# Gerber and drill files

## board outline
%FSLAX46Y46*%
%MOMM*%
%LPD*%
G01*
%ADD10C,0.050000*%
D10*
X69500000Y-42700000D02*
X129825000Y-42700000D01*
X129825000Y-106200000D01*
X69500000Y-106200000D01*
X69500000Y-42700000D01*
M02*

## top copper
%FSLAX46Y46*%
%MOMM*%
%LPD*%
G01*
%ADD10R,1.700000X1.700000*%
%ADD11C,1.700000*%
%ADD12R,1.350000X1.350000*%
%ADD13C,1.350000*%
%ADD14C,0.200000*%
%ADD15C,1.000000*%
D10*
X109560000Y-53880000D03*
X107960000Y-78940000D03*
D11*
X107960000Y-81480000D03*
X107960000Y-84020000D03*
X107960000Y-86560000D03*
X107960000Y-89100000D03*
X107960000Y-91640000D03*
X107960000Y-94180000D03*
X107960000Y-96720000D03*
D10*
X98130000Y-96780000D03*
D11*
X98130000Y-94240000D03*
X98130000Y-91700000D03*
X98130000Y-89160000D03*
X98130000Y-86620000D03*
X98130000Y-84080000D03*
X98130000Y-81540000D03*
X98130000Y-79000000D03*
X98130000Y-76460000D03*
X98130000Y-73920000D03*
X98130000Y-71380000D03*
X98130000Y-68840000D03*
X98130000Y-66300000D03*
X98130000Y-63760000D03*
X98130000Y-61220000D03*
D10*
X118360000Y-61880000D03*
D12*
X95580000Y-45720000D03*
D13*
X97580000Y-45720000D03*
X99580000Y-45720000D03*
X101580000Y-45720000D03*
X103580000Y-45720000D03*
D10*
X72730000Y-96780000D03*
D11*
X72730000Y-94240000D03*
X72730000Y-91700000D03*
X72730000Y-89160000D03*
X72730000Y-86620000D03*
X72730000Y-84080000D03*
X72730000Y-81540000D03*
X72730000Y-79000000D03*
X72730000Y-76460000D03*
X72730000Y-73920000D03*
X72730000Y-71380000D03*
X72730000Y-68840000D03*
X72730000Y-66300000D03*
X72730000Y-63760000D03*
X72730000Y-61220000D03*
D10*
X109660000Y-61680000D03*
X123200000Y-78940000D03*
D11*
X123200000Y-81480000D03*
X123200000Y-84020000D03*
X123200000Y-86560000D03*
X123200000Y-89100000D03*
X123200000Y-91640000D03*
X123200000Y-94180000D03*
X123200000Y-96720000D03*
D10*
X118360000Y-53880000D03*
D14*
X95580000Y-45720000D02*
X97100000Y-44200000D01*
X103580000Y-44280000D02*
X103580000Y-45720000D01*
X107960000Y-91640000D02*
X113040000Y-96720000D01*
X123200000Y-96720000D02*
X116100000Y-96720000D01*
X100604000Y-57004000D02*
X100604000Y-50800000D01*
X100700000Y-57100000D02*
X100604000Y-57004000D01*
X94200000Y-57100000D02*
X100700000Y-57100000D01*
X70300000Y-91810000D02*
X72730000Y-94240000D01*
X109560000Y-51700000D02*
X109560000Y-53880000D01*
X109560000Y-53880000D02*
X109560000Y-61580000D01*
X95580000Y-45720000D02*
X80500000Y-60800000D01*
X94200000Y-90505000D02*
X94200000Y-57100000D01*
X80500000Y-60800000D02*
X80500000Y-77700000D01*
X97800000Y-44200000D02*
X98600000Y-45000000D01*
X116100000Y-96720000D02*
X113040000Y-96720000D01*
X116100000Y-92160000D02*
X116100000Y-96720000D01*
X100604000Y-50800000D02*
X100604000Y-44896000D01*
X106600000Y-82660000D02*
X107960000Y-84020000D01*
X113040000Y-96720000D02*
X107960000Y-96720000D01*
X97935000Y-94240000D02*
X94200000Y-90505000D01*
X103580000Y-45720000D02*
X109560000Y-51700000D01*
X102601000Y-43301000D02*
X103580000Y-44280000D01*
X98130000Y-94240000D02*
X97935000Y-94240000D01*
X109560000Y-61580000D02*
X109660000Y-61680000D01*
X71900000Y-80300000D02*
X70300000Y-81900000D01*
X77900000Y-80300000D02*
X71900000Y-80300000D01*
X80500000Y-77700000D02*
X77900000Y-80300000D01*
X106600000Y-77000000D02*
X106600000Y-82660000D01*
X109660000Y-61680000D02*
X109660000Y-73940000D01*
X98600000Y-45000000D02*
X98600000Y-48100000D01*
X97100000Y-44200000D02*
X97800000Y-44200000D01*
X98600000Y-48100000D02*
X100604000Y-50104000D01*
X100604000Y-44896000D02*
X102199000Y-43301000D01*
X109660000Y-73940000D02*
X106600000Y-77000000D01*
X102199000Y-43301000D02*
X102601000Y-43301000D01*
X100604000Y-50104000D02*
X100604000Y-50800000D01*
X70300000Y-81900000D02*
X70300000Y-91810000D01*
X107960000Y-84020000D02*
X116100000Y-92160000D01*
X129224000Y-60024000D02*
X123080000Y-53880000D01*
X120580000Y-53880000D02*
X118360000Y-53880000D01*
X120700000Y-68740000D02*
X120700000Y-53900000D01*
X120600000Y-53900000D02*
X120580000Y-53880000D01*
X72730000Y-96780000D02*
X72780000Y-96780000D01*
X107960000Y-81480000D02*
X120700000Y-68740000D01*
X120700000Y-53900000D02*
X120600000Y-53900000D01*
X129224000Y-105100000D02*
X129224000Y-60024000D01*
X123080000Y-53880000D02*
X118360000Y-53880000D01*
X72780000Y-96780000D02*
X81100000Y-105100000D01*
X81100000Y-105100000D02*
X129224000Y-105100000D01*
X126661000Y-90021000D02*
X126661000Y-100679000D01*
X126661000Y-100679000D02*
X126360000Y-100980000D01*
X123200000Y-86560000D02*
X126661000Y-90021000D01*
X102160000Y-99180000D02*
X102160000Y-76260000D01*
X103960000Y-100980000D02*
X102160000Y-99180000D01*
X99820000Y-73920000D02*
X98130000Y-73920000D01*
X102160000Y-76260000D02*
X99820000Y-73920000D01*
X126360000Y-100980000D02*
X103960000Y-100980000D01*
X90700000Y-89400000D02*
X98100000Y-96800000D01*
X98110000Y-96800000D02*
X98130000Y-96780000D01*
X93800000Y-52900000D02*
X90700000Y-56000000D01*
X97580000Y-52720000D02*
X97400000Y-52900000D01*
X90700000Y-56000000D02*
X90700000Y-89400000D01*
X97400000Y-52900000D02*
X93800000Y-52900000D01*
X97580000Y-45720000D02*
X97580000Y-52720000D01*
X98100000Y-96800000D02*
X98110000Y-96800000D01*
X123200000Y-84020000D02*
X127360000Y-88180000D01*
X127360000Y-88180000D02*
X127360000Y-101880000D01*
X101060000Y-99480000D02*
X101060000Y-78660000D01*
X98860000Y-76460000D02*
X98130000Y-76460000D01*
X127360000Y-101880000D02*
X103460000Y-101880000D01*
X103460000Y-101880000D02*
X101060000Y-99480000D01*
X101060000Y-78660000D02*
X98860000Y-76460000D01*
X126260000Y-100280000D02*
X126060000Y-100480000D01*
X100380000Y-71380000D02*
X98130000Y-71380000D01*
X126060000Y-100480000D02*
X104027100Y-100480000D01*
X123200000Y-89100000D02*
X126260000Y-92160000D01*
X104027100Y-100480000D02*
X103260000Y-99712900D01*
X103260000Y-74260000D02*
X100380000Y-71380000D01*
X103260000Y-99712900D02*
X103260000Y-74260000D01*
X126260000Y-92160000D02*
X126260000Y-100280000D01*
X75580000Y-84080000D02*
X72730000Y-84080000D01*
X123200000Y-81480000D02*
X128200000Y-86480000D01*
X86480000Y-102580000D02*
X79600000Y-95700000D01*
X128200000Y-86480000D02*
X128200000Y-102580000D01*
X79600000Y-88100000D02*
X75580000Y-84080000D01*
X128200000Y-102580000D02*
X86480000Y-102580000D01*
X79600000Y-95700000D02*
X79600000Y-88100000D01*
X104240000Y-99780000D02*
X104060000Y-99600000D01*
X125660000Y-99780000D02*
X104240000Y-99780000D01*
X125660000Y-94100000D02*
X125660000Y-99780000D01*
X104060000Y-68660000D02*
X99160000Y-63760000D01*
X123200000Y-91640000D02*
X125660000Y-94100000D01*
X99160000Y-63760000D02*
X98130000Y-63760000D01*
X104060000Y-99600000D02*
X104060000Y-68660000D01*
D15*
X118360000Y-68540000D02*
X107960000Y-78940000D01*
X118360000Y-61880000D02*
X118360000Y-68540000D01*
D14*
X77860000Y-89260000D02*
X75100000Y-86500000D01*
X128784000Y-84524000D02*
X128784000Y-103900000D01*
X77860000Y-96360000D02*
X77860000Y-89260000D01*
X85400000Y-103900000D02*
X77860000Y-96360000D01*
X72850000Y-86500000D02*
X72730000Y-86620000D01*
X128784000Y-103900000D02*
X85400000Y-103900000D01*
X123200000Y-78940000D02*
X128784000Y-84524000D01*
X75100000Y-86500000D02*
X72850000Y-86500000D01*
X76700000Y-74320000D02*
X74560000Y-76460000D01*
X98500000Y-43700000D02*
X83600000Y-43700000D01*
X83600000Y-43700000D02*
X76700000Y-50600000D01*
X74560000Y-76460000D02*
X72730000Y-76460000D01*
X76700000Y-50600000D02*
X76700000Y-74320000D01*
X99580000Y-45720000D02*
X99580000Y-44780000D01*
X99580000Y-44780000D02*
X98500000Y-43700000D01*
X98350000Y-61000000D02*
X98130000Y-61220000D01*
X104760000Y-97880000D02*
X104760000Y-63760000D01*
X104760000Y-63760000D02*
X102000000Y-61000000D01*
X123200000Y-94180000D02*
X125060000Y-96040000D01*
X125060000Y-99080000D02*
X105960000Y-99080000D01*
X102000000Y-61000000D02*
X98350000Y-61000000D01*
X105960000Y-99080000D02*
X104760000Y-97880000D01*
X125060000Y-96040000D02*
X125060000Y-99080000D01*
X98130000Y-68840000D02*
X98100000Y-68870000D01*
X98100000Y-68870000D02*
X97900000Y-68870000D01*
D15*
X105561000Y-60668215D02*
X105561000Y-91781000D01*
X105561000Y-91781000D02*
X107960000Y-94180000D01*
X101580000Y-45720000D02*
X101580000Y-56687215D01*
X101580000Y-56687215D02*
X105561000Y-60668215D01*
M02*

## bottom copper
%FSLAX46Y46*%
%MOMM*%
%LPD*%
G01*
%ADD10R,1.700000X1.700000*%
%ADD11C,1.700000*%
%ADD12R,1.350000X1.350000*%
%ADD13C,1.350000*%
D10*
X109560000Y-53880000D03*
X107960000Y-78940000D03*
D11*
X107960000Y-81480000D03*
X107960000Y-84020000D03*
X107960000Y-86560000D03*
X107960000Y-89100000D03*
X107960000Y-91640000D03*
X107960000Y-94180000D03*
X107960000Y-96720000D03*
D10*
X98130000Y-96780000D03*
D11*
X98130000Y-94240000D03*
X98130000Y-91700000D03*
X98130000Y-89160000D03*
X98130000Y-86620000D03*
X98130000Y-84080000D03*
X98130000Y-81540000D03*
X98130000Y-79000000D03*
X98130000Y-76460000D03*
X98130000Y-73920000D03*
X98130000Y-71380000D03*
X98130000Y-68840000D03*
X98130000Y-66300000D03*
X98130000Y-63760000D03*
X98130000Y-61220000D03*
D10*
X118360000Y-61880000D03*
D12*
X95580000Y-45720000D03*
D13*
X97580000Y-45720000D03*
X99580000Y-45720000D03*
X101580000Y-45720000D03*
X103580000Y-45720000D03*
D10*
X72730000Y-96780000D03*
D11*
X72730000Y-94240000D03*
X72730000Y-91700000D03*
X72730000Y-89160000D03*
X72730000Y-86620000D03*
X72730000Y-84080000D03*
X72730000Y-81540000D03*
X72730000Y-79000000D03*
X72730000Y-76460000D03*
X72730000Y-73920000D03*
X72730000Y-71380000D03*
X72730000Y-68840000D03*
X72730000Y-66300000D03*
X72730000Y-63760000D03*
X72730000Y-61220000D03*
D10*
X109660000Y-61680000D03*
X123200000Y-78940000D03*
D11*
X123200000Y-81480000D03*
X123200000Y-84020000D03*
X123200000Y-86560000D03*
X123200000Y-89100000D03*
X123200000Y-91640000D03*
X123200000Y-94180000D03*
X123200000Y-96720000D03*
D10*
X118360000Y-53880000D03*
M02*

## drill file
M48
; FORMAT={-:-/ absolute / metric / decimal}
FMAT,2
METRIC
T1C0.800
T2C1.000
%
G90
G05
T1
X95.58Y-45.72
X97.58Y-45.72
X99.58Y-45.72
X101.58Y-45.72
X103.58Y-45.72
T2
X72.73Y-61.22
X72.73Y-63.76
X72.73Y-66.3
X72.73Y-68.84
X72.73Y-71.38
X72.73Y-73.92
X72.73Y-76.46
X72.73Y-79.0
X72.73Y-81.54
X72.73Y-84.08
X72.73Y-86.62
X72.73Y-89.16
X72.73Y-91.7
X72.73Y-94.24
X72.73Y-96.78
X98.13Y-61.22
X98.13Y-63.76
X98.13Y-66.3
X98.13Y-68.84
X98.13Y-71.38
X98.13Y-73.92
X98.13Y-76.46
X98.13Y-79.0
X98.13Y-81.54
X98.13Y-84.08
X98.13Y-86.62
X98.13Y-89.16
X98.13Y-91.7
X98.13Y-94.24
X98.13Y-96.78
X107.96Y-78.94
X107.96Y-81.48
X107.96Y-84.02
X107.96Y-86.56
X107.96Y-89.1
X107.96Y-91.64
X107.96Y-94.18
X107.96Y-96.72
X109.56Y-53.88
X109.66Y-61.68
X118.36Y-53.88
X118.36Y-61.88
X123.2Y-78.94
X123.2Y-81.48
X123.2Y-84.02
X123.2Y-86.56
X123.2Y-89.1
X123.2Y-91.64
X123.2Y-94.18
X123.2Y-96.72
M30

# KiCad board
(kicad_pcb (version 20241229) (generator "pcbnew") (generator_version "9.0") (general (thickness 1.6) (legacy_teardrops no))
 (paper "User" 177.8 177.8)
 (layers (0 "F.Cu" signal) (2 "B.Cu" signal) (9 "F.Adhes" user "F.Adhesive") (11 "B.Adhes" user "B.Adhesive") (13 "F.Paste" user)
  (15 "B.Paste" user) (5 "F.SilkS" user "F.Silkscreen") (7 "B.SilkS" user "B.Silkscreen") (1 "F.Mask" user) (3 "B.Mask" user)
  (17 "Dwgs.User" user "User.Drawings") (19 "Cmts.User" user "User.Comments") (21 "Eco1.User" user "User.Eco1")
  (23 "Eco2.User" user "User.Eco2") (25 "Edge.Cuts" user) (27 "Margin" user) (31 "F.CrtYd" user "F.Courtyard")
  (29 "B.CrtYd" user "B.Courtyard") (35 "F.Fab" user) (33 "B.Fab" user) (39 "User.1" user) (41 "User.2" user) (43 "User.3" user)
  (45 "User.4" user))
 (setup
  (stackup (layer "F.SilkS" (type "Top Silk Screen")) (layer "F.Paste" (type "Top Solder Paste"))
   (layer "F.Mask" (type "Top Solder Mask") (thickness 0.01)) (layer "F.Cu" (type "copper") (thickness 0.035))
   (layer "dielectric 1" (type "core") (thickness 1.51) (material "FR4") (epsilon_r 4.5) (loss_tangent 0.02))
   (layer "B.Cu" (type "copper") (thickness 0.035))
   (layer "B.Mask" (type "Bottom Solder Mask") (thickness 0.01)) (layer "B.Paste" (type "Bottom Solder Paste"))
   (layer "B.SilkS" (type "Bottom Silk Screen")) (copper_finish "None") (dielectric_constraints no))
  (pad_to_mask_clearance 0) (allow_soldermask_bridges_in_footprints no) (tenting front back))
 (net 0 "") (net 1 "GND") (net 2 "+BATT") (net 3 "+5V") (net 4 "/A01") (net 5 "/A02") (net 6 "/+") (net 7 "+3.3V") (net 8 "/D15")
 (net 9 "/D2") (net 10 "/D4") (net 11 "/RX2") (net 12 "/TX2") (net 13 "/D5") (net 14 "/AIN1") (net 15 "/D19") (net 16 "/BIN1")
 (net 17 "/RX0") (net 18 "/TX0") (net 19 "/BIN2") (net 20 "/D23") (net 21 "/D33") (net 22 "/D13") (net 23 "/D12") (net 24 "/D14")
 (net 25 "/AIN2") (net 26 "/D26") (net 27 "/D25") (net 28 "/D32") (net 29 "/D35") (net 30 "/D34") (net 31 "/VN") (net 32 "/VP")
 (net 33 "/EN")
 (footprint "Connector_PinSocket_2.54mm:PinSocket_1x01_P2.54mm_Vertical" (layer "F.Cu") (at 109.56 53.88)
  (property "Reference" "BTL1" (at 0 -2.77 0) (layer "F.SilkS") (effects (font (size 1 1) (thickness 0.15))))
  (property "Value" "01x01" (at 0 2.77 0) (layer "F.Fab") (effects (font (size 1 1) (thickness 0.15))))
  (pad "1" thru_hole rect (at 0 0) (size 1.7 1.7) (drill 1) (layers "*.Cu" "*.Mask") (remove_unused_layers no) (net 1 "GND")))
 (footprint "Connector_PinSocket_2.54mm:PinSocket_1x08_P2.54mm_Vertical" (layer "F.Cu") (at 107.96 78.94)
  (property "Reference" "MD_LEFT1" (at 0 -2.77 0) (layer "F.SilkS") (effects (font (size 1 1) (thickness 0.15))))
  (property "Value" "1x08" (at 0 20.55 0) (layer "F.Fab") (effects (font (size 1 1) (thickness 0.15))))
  (pad "1" thru_hole rect (at 0 0) (size 1.7 1.7) (drill 1) (layers "*.Cu" "*.Mask") (remove_unused_layers no) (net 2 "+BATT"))
  (pad "2" thru_hole circle (at 0 2.54) (size 1.7 1.7) (drill 1) (layers "*.Cu" "*.Mask") (remove_unused_layers no) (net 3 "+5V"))
  (pad "3" thru_hole circle (at 0 5.08) (size 1.7 1.7) (drill 1) (layers "*.Cu" "*.Mask") (remove_unused_layers no) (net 1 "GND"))
  (pad "4" thru_hole circle (at 0 7.62) (size 1.7 1.7) (drill 1) (layers "*.Cu" "*.Mask") (remove_unused_layers no) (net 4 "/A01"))
  (pad "5" thru_hole circle (at 0 10.16) (size 1.7 1.7) (drill 1) (layers "*.Cu" "*.Mask") (remove_unused_layers no) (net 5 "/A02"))
  (pad "6" thru_hole circle (at 0 12.7) (size 1.7 1.7) (drill 1) (layers "*.Cu" "*.Mask") (remove_unused_layers no) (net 1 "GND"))
  (pad "7" thru_hole circle (at 0 15.24) (size 1.7 1.7) (drill 1) (layers "*.Cu" "*.Mask") (remove_unused_layers no) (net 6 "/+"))
  (pad "8" thru_hole circle (at 0 17.78) (size 1.7 1.7) (drill 1) (layers "*.Cu" "*.Mask") (remove_unused_layers no) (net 1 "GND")))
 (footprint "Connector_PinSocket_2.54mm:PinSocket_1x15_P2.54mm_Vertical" (layer "F.Cu") (at 98.13 96.78 180)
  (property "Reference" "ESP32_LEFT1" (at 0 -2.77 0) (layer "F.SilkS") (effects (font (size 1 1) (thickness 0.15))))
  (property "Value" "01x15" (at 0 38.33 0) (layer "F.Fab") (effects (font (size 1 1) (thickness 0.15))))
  (pad "1" thru_hole rect (at 0 0 180) (size 1.7 1.7) (drill 1) (layers "*.Cu" "*.Mask") (remove_unused_layers no) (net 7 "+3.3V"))
  (pad "2" thru_hole circle (at 0 2.54 180) (size 1.7 1.7) (drill 1) (layers "*.Cu" "*.Mask") (remove_unused_layers no) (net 1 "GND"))
  (pad "3" thru_hole circle (at 0 5.08 180) (size 1.7 1.7) (drill 1) (layers "*.Cu" "*.Mask") (remove_unused_layers no) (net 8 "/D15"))
  (pad "4" thru_hole circle (at 0 7.62 180) (size 1.7 1.7) (drill 1) (layers "*.Cu" "*.Mask") (remove_unused_layers no) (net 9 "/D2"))
  (pad "5" thru_hole circle (at 0 10.16 180) (size 1.7 1.7) (drill 1) (layers "*.Cu" "*.Mask") (remove_unused_layers no) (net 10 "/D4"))
  (pad "6" thru_hole circle (at 0 12.7 180) (size 1.7 1.7) (drill 1) (layers "*.Cu" "*.Mask") (remove_unused_layers no) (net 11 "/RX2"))
  (pad "7" thru_hole circle (at 0 15.24 180) (size 1.7 1.7) (drill 1) (layers "*.Cu" "*.Mask") (remove_unused_layers no) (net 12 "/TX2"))
  (pad "8" thru_hole circle (at 0 17.78 180) (size 1.7 1.7) (drill 1) (layers "*.Cu" "*.Mask") (remove_unused_layers no) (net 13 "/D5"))
  (pad "9" thru_hole circle (at 0 20.32 180) (size 1.7 1.7) (drill 1) (layers "*.Cu" "*.Mask") (remove_unused_layers no) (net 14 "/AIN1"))
  (pad "10" thru_hole circle (at 0 22.86 180) (size 1.7 1.7) (drill 1) (layers "*.Cu" "*.Mask") (remove_unused_layers no) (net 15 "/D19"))
  (pad "11" thru_hole circle (at 0 25.4 180) (size 1.7 1.7) (drill 1) (layers "*.Cu" "*.Mask") (remove_unused_layers no) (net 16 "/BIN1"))
  (pad "12" thru_hole circle (at 0 27.94 180) (size 1.7 1.7) (drill 1) (layers "*.Cu" "*.Mask") (remove_unused_layers no) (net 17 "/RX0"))
  (pad "13" thru_hole circle (at 0 30.48 180) (size 1.7 1.7) (drill 1) (layers "*.Cu" "*.Mask") (remove_unused_layers no) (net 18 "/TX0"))
  (pad "14" thru_hole circle (at 0 33.02 180) (size 1.7 1.7) (drill 1) (layers "*.Cu" "*.Mask") (remove_unused_layers no) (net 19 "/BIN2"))
  (pad "15" thru_hole circle (at 0 35.56 180) (size 1.7 1.7) (drill 1) (layers "*.Cu" "*.Mask") (remove_unused_layers no) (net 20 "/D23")))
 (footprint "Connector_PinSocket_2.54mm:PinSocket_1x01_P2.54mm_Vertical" (layer "F.Cu") (at 118.36 61.88)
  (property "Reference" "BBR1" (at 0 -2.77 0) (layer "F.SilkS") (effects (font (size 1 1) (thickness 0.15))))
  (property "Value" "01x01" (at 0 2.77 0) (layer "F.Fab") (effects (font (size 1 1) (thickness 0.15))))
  (pad "1" thru_hole rect (at 0 0) (size 1.7 1.7) (drill 1) (layers "*.Cu" "*.Mask") (remove_unused_layers no) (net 2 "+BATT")))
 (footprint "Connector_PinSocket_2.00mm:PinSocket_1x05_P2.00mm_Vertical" (layer "F.Cu") (at 95.58 45.72 90)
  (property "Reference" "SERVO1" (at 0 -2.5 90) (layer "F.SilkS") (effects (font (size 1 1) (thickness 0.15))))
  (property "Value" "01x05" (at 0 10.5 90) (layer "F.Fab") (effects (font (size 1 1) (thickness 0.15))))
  (pad "1" thru_hole rect (at 0 0 90) (size 1.35 1.35) (drill 0.8) (layers "*.Cu" "*.Mask") (remove_unused_layers no) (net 1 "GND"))
  (pad "2" thru_hole circle (at 0 2 90) (size 1.35 1.35) (drill 0.8) (layers "*.Cu" "*.Mask") (remove_unused_layers no) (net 7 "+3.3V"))
  (pad "3" thru_hole circle (at 0 4 90) (size 1.35 1.35) (drill 0.8) (layers "*.Cu" "*.Mask") (remove_unused_layers no) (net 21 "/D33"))
  (pad "4" thru_hole circle (at 0 6 90) (size 1.35 1.35) (drill 0.8) (layers "*.Cu" "*.Mask") (remove_unused_layers no) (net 6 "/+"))
  (pad "5" thru_hole circle (at 0 8 90) (size 1.35 1.35) (drill 0.8) (layers "*.Cu" "*.Mask") (remove_unused_layers no) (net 1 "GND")))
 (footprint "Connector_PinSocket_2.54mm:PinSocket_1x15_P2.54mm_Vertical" (layer "F.Cu") (at 72.73 96.78 180)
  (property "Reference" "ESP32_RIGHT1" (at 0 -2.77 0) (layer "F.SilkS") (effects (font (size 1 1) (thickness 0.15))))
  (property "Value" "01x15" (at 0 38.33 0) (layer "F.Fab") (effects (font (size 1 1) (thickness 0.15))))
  (pad "1" thru_hole rect (at 0 0 180) (size 1.7 1.7) (drill 1) (layers "*.Cu" "*.Mask") (remove_unused_layers no) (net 3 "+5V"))
  (pad "2" thru_hole circle (at 0 2.54 180) (size 1.7 1.7) (drill 1) (layers "*.Cu" "*.Mask") (remove_unused_layers no) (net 1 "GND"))
  (pad "3" thru_hole circle (at 0 5.08 180) (size 1.7 1.7) (drill 1) (layers "*.Cu" "*.Mask") (remove_unused_layers no) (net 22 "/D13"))
  (pad "4" thru_hole circle (at 0 7.62 180) (size 1.7 1.7) (drill 1) (layers "*.Cu" "*.Mask") (remove_unused_layers no) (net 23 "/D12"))
  (pad "5" thru_hole circle (at 0 10.16 180) (size 1.7 1.7) (drill 1) (layers "*.Cu" "*.Mask") (remove_unused_layers no) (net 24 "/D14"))
  (pad "6" thru_hole circle (at 0 12.7 180) (size 1.7 1.7) (drill 1) (layers "*.Cu" "*.Mask") (remove_unused_layers no) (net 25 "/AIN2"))
  (pad "7" thru_hole circle (at 0 15.24 180) (size 1.7 1.7) (drill 1) (layers "*.Cu" "*.Mask") (remove_unused_layers no) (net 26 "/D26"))
  (pad "8" thru_hole circle (at 0 17.78 180) (size 1.7 1.7) (drill 1) (layers "*.Cu" "*.Mask") (remove_unused_layers no) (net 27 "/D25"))
  (pad "9" thru_hole circle (at 0 20.32 180) (size 1.7 1.7) (drill 1) (layers "*.Cu" "*.Mask") (remove_unused_layers no) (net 21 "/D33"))
  (pad "10" thru_hole circle (at 0 22.86 180) (size 1.7 1.7) (drill 1) (layers "*.Cu" "*.Mask") (remove_unused_layers no) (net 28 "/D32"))
  (pad "11" thru_hole circle (at 0 25.4 180) (size 1.7 1.7) (drill 1) (layers "*.Cu" "*.Mask") (remove_unused_layers no) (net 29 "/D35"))
  (pad "12" thru_hole circle (at 0 27.94 180) (size 1.7 1.7) (drill 1) (layers "*.Cu" "*.Mask") (remove_unused_layers no) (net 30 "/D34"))
  (pad "13" thru_hole circle (at 0 30.48 180) (size 1.7 1.7) (drill 1) (layers "*.Cu" "*.Mask") (remove_unused_layers no) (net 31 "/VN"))
  (pad "14" thru_hole circle (at 0 33.02 180) (size 1.7 1.7) (drill 1) (layers "*.Cu" "*.Mask") (remove_unused_layers no) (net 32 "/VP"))
  (pad "15" thru_hole circle (at 0 35.56 180) (size 1.7 1.7) (drill 1) (layers "*.Cu" "*.Mask") (remove_unused_layers no) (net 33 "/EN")))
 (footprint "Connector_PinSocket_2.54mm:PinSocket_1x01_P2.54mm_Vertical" (layer "F.Cu") (at 109.66 61.68)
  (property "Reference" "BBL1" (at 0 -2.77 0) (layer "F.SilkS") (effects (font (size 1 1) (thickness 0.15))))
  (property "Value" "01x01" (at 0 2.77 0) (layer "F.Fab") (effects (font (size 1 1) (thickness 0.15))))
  (pad "1" thru_hole rect (at 0 0) (size 1.7 1.7) (drill 1) (layers "*.Cu" "*.Mask") (remove_unused_layers no) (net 1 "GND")))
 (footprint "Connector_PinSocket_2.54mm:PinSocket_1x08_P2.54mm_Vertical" (layer "F.Cu") (at 123.2 78.94)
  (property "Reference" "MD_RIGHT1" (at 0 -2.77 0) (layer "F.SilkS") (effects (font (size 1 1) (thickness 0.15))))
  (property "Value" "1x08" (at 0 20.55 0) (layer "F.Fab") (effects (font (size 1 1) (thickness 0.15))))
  (pad "1" thru_hole rect (at 0 0) (size 1.7 1.7) (drill 1) (layers "*.Cu" "*.Mask") (remove_unused_layers no) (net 24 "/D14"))
  (pad "2" thru_hole circle (at 0 2.54) (size 1.7 1.7) (drill 1) (layers "*.Cu" "*.Mask") (remove_unused_layers no) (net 25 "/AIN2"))
  (pad "3" thru_hole circle (at 0 5.08) (size 1.7 1.7) (drill 1) (layers "*.Cu" "*.Mask") (remove_unused_layers no) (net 14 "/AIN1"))
  (pad "4" thru_hole circle (at 0 7.62) (size 1.7 1.7) (drill 1) (layers "*.Cu" "*.Mask") (remove_unused_layers no) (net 15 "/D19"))
  (pad "5" thru_hole circle (at 0 10.16) (size 1.7 1.7) (drill 1) (layers "*.Cu" "*.Mask") (remove_unused_layers no) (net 16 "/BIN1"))
  (pad "6" thru_hole circle (at 0 12.7) (size 1.7 1.7) (drill 1) (layers "*.Cu" "*.Mask") (remove_unused_layers no) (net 19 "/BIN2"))
  (pad "7" thru_hole circle (at 0 15.24) (size 1.7 1.7) (drill 1) (layers "*.Cu" "*.Mask") (remove_unused_layers no) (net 20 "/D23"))
  (pad "8" thru_hole circle (at 0 17.78) (size 1.7 1.7) (drill 1) (layers "*.Cu" "*.Mask") (remove_unused_layers no) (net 1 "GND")))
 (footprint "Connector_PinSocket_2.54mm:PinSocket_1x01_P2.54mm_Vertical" (layer "F.Cu") (at 118.36 53.88)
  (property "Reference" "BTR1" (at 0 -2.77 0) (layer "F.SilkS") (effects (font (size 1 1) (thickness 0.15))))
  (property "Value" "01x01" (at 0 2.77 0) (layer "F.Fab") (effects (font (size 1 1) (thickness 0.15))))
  (pad "1" thru_hole rect (at 0 0) (size 1.7 1.7) (drill 1) (layers "*.Cu" "*.Mask") (remove_unused_layers no) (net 3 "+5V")))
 (gr_rect (start 69.5 42.7) (end 129.825 106.2) (stroke (width 0.05) (type solid)) (fill no) (layer "Edge.Cuts"))
 (segment (start 95.58 45.72) (end 97.1 44.2) (width 0.2) (layer "F.Cu") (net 1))
 (segment (start 103.58 44.28) (end 103.58 45.72) (width 0.2) (layer "F.Cu") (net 1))
 (segment (start 107.96 91.64) (end 113.04 96.72) (width 0.2) (layer "F.Cu") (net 1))
 (segment (start 123.2 96.72) (end 116.1 96.72) (width 0.2) (layer "F.Cu") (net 1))
 (segment (start 100.604 57.004) (end 100.604 50.8) (width 0.2) (layer "F.Cu") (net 1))
 (segment (start 100.7 57.1) (end 100.604 57.004) (width 0.2) (layer "F.Cu") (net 1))
 (segment (start 94.2 57.1) (end 100.7 57.1) (width 0.2) (layer "F.Cu") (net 1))
 (segment (start 70.3 91.81) (end 72.73 94.24) (width 0.2) (layer "F.Cu") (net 1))
 (segment (start 109.56 51.7) (end 109.56 53.88) (width 0.2) (layer "F.Cu") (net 1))
 (segment (start 109.56 53.88) (end 109.56 61.58) (width 0.2) (layer "F.Cu") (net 1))
 (segment (start 95.58 45.72) (end 80.5 60.8) (width 0.2) (layer "F.Cu") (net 1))
 (segment (start 94.2 90.505) (end 94.2 57.1) (width 0.2) (layer "F.Cu") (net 1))
 (segment (start 80.5 60.8) (end 80.5 77.7) (width 0.2) (layer "F.Cu") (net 1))
 (segment (start 97.8 44.2) (end 98.6 45) (width 0.2) (layer "F.Cu") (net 1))
 (segment (start 116.1 96.72) (end 113.04 96.72) (width 0.2) (layer "F.Cu") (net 1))
 (segment (start 116.1 92.16) (end 116.1 96.72) (width 0.2) (layer "F.Cu") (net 1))
 (segment (start 100.604 50.8) (end 100.604 44.896) (width 0.2) (layer "F.Cu") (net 1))
 (segment (start 106.6 82.66) (end 107.96 84.02) (width 0.2) (layer "F.Cu") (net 1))
 (segment (start 113.04 96.72) (end 107.96 96.72) (width 0.2) (layer "F.Cu") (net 1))
 (segment (start 97.935 94.24) (end 94.2 90.505) (width 0.2) (layer "F.Cu") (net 1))
 (segment (start 103.58 45.72) (end 109.56 51.7) (width 0.2) (layer "F.Cu") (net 1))
 (segment (start 102.601 43.301) (end 103.58 44.28) (width 0.2) (layer "F.Cu") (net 1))
 (segment (start 98.13 94.24) (end 97.935 94.24) (width 0.2) (layer "F.Cu") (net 1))
 (segment (start 109.56 61.58) (end 109.66 61.68) (width 0.2) (layer "F.Cu") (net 1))
 (segment (start 71.9 80.3) (end 70.3 81.9) (width 0.2) (layer "F.Cu") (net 1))
 (segment (start 77.9 80.3) (end 71.9 80.3) (width 0.2) (layer "F.Cu") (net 1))
 (segment (start 80.5 77.7) (end 77.9 80.3) (width 0.2) (layer "F.Cu") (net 1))
 (segment (start 106.6 77) (end 106.6 82.66) (width 0.2) (layer "F.Cu") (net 1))
 (segment (start 109.66 61.68) (end 109.66 73.94) (width 0.2) (layer "F.Cu") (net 1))
 (segment (start 98.6 45) (end 98.6 48.1) (width 0.2) (layer "F.Cu") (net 1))
 (segment (start 97.1 44.2) (end 97.8 44.2) (width 0.2) (layer "F.Cu") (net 1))
 (segment (start 98.6 48.1) (end 100.604 50.104) (width 0.2) (layer "F.Cu") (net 1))
 (segment (start 100.604 44.896) (end 102.199 43.301) (width 0.2) (layer "F.Cu") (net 1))
 (segment (start 109.66 73.94) (end 106.6 77) (width 0.2) (layer "F.Cu") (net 1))
 (segment (start 102.199 43.301) (end 102.601 43.301) (width 0.2) (layer "F.Cu") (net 1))
 (segment (start 100.604 50.104) (end 100.604 50.8) (width 0.2) (layer "F.Cu") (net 1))
 (segment (start 70.3 81.9) (end 70.3 91.81) (width 0.2) (layer "F.Cu") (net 1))
 (segment (start 107.96 84.02) (end 116.1 92.16) (width 0.2) (layer "F.Cu") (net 1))
 (segment (start 129.224 60.024) (end 123.08 53.88) (width 0.2) (layer "F.Cu") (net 3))
 (segment (start 120.58 53.88) (end 118.36 53.88) (width 0.2) (layer "F.Cu") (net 3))
 (segment (start 120.7 68.74) (end 120.7 53.9) (width 0.2) (layer "F.Cu") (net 3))
 (segment (start 120.6 53.9) (end 120.58 53.88) (width 0.2) (layer "F.Cu") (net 3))
 (segment (start 72.73 96.78) (end 72.78 96.78) (width 0.2) (layer "F.Cu") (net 3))
 (segment (start 107.96 81.48) (end 120.7 68.74) (width 0.2) (layer "F.Cu") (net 3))
 (segment (start 120.7 53.9) (end 120.6 53.9) (width 0.2) (layer "F.Cu") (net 3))
 (segment (start 129.224 105.1) (end 129.224 60.024) (width 0.2) (layer "F.Cu") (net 3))
 (segment (start 123.08 53.88) (end 118.36 53.88) (width 0.2) (layer "F.Cu") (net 3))
 (segment (start 72.78 96.78) (end 81.1 105.1) (width 0.2) (layer "F.Cu") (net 3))
 (segment (start 81.1 105.1) (end 129.224 105.1) (width 0.2) (layer "F.Cu") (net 3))
 (segment (start 126.661 90.021) (end 126.661 100.679) (width 0.2) (layer "F.Cu") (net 15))
 (segment (start 126.661 100.679) (end 126.36 100.98) (width 0.2) (layer "F.Cu") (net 15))
 (segment (start 123.2 86.56) (end 126.661 90.021) (width 0.2) (layer "F.Cu") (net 15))
 (segment (start 102.16 99.18) (end 102.16 76.26) (width 0.2) (layer "F.Cu") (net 15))
 (segment (start 103.96 100.98) (end 102.16 99.18) (width 0.2) (layer "F.Cu") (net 15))
 (segment (start 99.82 73.92) (end 98.13 73.92) (width 0.2) (layer "F.Cu") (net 15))
 (segment (start 102.16 76.26) (end 99.82 73.92) (width 0.2) (layer "F.Cu") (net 15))
 (segment (start 126.36 100.98) (end 103.96 100.98) (width 0.2) (layer "F.Cu") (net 15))
 (segment (start 90.7 89.4) (end 98.1 96.8) (width 0.2) (layer "F.Cu") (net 7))
 (segment (start 98.11 96.8) (end 98.13 96.78) (width 0.2) (layer "F.Cu") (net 7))
 (segment (start 93.8 52.9) (end 90.7 56) (width 0.2) (layer "F.Cu") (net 7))
 (segment (start 97.58 52.72) (end 97.4 52.9) (width 0.2) (layer "F.Cu") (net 7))
 (segment (start 90.7 56) (end 90.7 89.4) (width 0.2) (layer "F.Cu") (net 7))
 (segment (start 97.4 52.9) (end 93.8 52.9) (width 0.2) (layer "F.Cu") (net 7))
 (segment (start 97.58 45.72) (end 97.58 52.72) (width 0.2) (layer "F.Cu") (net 7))
 (segment (start 98.1 96.8) (end 98.11 96.8) (width 0.2) (layer "F.Cu") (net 7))
 (segment (start 123.2 84.02) (end 127.36 88.18) (width 0.2) (layer "F.Cu") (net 14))
 (segment (start 127.36 88.18) (end 127.36 101.88) (width 0.2) (layer "F.Cu") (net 14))
 (segment (start 101.06 99.48) (end 101.06 78.66) (width 0.2) (layer "F.Cu") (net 14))
 (segment (start 98.86 76.46) (end 98.13 76.46) (width 0.2) (layer "F.Cu") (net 14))
 (segment (start 127.36 101.88) (end 103.46 101.88) (width 0.2) (layer "F.Cu") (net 14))
 (segment (start 103.46 101.88) (end 101.06 99.48) (width 0.2) (layer "F.Cu") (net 14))
 (segment (start 101.06 78.66) (end 98.86 76.46) (width 0.2) (layer "F.Cu") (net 14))
 (segment (start 126.26 100.28) (end 126.06 100.48) (width 0.2) (layer "F.Cu") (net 16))
 (segment (start 100.38 71.38) (end 98.13 71.38) (width 0.2) (layer "F.Cu") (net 16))
 (segment (start 126.06 100.48) (end 104.0271 100.48) (width 0.2) (layer "F.Cu") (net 16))
 (segment (start 123.2 89.1) (end 126.26 92.16) (width 0.2) (layer "F.Cu") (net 16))
 (segment (start 104.0271 100.48) (end 103.26 99.7129) (width 0.2) (layer "F.Cu") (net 16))
 (segment (start 103.26 74.26) (end 100.38 71.38) (width 0.2) (layer "F.Cu") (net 16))
 (segment (start 103.26 99.7129) (end 103.26 74.26) (width 0.2) (layer "F.Cu") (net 16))
 (segment (start 126.26 92.16) (end 126.26 100.28) (width 0.2) (layer "F.Cu") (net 16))
 (segment (start 75.58 84.08) (end 72.73 84.08) (width 0.2) (layer "F.Cu") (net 25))
 (segment (start 123.2 81.48) (end 128.2 86.48) (width 0.2) (layer "F.Cu") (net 25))
 (segment (start 86.48 102.58) (end 79.6 95.7) (width 0.2) (layer "F.Cu") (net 25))
 (segment (start 128.2 86.48) (end 128.2 102.58) (width 0.2) (layer "F.Cu") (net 25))
 (segment (start 79.6 88.1) (end 75.58 84.08) (width 0.2) (layer "F.Cu") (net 25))
 (segment (start 128.2 102.58) (end 86.48 102.58) (width 0.2) (layer "F.Cu") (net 25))
 (segment (start 79.6 95.7) (end 79.6 88.1) (width 0.2) (layer "F.Cu") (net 25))
 (segment (start 104.24 99.78) (end 104.06 99.6) (width 0.2) (layer "F.Cu") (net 19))
 (segment (start 125.66 99.78) (end 104.24 99.78) (width 0.2) (layer "F.Cu") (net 19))
 (segment (start 125.66 94.1) (end 125.66 99.78) (width 0.2) (layer "F.Cu") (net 19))
 (segment (start 104.06 68.66) (end 99.16 63.76) (width 0.2) (layer "F.Cu") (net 19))
 (segment (start 123.2 91.64) (end 125.66 94.1) (width 0.2) (layer "F.Cu") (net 19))
 (segment (start 99.16 63.76) (end 98.13 63.76) (width 0.2) (layer "F.Cu") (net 19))
 (segment (start 104.06 99.6) (end 104.06 68.66) (width 0.2) (layer "F.Cu") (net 19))
 (segment (start 118.36 68.54) (end 107.96 78.94) (width 1) (layer "F.Cu") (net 2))
 (segment (start 118.36 61.88) (end 118.36 68.54) (width 1) (layer "F.Cu") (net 2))
 (segment (start 77.86 89.26) (end 75.1 86.5) (width 0.2) (layer "F.Cu") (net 24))
 (segment (start 128.784 84.524) (end 128.784 103.9) (width 0.2) (layer "F.Cu") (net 24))
 (segment (start 77.86 96.36) (end 77.86 89.26) (width 0.2) (layer "F.Cu") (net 24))
 (segment (start 85.4 103.9) (end 77.86 96.36) (width 0.2) (layer "F.Cu") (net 24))
 (segment (start 72.85 86.5) (end 72.73 86.62) (width 0.2) (layer "F.Cu") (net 24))
 (segment (start 128.784 103.9) (end 85.4 103.9) (width 0.2) (layer "F.Cu") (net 24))
 (segment (start 123.2 78.94) (end 128.784 84.524) (width 0.2) (layer "F.Cu") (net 24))
 (segment (start 75.1 86.5) (end 72.85 86.5) (width 0.2) (layer "F.Cu") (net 24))
 (segment (start 76.7 74.32) (end 74.56 76.46) (width 0.2) (layer "F.Cu") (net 21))
 (segment (start 98.5 43.7) (end 83.6 43.7) (width 0.2) (layer "F.Cu") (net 21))
 (segment (start 83.6 43.7) (end 76.7 50.6) (width 0.2) (layer "F.Cu") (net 21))
 (segment (start 74.56 76.46) (end 72.73 76.46) (width 0.2) (layer "F.Cu") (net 21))
 (segment (start 76.7 50.6) (end 76.7 74.32) (width 0.2) (layer "F.Cu") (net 21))
 (segment (start 99.58 45.72) (end 99.58 44.78) (width 0.2) (layer "F.Cu") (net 21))
 (segment (start 99.58 44.78) (end 98.5 43.7) (width 0.2) (layer "F.Cu") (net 21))
 (segment (start 98.35 61) (end 98.13 61.22) (width 0.2) (layer "F.Cu") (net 20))
 (segment (start 104.76 97.88) (end 104.76 63.76) (width 0.2) (layer "F.Cu") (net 20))
 (segment (start 104.76 63.76) (end 102 61) (width 0.2) (layer "F.Cu") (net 20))
 (segment (start 123.2 94.18) (end 125.06 96.04) (width 0.2) (layer "F.Cu") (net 20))
 (segment (start 125.06 99.08) (end 105.96 99.08) (width 0.2) (layer "F.Cu") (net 20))
 (segment (start 102 61) (end 98.35 61) (width 0.2) (layer "F.Cu") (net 20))
 (segment (start 105.96 99.08) (end 104.76 97.88) (width 0.2) (layer "F.Cu") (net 20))
 (segment (start 125.06 96.04) (end 125.06 99.08) (width 0.2) (layer "F.Cu") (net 20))
 (segment (start 98.13 68.84) (end 98.1 68.87) (width 0.2) (layer "F.Cu") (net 17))
 (segment (start 98.1 68.87) (end 97.9 68.87) (width 0.2) (layer "F.Cu") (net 17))
 (segment (start 105.561 60.668215) (end 105.561 91.781) (width 1) (layer "F.Cu") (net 6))
 (segment (start 105.561 91.781) (end 107.96 94.18) (width 1) (layer "F.Cu") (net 6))
 (segment (start 101.58 45.72) (end 101.58 56.687215) (width 1) (layer "F.Cu") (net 6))
 (segment (start 101.58 56.687215) (end 105.561 60.668215) (width 1) (layer "F.Cu") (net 6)))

